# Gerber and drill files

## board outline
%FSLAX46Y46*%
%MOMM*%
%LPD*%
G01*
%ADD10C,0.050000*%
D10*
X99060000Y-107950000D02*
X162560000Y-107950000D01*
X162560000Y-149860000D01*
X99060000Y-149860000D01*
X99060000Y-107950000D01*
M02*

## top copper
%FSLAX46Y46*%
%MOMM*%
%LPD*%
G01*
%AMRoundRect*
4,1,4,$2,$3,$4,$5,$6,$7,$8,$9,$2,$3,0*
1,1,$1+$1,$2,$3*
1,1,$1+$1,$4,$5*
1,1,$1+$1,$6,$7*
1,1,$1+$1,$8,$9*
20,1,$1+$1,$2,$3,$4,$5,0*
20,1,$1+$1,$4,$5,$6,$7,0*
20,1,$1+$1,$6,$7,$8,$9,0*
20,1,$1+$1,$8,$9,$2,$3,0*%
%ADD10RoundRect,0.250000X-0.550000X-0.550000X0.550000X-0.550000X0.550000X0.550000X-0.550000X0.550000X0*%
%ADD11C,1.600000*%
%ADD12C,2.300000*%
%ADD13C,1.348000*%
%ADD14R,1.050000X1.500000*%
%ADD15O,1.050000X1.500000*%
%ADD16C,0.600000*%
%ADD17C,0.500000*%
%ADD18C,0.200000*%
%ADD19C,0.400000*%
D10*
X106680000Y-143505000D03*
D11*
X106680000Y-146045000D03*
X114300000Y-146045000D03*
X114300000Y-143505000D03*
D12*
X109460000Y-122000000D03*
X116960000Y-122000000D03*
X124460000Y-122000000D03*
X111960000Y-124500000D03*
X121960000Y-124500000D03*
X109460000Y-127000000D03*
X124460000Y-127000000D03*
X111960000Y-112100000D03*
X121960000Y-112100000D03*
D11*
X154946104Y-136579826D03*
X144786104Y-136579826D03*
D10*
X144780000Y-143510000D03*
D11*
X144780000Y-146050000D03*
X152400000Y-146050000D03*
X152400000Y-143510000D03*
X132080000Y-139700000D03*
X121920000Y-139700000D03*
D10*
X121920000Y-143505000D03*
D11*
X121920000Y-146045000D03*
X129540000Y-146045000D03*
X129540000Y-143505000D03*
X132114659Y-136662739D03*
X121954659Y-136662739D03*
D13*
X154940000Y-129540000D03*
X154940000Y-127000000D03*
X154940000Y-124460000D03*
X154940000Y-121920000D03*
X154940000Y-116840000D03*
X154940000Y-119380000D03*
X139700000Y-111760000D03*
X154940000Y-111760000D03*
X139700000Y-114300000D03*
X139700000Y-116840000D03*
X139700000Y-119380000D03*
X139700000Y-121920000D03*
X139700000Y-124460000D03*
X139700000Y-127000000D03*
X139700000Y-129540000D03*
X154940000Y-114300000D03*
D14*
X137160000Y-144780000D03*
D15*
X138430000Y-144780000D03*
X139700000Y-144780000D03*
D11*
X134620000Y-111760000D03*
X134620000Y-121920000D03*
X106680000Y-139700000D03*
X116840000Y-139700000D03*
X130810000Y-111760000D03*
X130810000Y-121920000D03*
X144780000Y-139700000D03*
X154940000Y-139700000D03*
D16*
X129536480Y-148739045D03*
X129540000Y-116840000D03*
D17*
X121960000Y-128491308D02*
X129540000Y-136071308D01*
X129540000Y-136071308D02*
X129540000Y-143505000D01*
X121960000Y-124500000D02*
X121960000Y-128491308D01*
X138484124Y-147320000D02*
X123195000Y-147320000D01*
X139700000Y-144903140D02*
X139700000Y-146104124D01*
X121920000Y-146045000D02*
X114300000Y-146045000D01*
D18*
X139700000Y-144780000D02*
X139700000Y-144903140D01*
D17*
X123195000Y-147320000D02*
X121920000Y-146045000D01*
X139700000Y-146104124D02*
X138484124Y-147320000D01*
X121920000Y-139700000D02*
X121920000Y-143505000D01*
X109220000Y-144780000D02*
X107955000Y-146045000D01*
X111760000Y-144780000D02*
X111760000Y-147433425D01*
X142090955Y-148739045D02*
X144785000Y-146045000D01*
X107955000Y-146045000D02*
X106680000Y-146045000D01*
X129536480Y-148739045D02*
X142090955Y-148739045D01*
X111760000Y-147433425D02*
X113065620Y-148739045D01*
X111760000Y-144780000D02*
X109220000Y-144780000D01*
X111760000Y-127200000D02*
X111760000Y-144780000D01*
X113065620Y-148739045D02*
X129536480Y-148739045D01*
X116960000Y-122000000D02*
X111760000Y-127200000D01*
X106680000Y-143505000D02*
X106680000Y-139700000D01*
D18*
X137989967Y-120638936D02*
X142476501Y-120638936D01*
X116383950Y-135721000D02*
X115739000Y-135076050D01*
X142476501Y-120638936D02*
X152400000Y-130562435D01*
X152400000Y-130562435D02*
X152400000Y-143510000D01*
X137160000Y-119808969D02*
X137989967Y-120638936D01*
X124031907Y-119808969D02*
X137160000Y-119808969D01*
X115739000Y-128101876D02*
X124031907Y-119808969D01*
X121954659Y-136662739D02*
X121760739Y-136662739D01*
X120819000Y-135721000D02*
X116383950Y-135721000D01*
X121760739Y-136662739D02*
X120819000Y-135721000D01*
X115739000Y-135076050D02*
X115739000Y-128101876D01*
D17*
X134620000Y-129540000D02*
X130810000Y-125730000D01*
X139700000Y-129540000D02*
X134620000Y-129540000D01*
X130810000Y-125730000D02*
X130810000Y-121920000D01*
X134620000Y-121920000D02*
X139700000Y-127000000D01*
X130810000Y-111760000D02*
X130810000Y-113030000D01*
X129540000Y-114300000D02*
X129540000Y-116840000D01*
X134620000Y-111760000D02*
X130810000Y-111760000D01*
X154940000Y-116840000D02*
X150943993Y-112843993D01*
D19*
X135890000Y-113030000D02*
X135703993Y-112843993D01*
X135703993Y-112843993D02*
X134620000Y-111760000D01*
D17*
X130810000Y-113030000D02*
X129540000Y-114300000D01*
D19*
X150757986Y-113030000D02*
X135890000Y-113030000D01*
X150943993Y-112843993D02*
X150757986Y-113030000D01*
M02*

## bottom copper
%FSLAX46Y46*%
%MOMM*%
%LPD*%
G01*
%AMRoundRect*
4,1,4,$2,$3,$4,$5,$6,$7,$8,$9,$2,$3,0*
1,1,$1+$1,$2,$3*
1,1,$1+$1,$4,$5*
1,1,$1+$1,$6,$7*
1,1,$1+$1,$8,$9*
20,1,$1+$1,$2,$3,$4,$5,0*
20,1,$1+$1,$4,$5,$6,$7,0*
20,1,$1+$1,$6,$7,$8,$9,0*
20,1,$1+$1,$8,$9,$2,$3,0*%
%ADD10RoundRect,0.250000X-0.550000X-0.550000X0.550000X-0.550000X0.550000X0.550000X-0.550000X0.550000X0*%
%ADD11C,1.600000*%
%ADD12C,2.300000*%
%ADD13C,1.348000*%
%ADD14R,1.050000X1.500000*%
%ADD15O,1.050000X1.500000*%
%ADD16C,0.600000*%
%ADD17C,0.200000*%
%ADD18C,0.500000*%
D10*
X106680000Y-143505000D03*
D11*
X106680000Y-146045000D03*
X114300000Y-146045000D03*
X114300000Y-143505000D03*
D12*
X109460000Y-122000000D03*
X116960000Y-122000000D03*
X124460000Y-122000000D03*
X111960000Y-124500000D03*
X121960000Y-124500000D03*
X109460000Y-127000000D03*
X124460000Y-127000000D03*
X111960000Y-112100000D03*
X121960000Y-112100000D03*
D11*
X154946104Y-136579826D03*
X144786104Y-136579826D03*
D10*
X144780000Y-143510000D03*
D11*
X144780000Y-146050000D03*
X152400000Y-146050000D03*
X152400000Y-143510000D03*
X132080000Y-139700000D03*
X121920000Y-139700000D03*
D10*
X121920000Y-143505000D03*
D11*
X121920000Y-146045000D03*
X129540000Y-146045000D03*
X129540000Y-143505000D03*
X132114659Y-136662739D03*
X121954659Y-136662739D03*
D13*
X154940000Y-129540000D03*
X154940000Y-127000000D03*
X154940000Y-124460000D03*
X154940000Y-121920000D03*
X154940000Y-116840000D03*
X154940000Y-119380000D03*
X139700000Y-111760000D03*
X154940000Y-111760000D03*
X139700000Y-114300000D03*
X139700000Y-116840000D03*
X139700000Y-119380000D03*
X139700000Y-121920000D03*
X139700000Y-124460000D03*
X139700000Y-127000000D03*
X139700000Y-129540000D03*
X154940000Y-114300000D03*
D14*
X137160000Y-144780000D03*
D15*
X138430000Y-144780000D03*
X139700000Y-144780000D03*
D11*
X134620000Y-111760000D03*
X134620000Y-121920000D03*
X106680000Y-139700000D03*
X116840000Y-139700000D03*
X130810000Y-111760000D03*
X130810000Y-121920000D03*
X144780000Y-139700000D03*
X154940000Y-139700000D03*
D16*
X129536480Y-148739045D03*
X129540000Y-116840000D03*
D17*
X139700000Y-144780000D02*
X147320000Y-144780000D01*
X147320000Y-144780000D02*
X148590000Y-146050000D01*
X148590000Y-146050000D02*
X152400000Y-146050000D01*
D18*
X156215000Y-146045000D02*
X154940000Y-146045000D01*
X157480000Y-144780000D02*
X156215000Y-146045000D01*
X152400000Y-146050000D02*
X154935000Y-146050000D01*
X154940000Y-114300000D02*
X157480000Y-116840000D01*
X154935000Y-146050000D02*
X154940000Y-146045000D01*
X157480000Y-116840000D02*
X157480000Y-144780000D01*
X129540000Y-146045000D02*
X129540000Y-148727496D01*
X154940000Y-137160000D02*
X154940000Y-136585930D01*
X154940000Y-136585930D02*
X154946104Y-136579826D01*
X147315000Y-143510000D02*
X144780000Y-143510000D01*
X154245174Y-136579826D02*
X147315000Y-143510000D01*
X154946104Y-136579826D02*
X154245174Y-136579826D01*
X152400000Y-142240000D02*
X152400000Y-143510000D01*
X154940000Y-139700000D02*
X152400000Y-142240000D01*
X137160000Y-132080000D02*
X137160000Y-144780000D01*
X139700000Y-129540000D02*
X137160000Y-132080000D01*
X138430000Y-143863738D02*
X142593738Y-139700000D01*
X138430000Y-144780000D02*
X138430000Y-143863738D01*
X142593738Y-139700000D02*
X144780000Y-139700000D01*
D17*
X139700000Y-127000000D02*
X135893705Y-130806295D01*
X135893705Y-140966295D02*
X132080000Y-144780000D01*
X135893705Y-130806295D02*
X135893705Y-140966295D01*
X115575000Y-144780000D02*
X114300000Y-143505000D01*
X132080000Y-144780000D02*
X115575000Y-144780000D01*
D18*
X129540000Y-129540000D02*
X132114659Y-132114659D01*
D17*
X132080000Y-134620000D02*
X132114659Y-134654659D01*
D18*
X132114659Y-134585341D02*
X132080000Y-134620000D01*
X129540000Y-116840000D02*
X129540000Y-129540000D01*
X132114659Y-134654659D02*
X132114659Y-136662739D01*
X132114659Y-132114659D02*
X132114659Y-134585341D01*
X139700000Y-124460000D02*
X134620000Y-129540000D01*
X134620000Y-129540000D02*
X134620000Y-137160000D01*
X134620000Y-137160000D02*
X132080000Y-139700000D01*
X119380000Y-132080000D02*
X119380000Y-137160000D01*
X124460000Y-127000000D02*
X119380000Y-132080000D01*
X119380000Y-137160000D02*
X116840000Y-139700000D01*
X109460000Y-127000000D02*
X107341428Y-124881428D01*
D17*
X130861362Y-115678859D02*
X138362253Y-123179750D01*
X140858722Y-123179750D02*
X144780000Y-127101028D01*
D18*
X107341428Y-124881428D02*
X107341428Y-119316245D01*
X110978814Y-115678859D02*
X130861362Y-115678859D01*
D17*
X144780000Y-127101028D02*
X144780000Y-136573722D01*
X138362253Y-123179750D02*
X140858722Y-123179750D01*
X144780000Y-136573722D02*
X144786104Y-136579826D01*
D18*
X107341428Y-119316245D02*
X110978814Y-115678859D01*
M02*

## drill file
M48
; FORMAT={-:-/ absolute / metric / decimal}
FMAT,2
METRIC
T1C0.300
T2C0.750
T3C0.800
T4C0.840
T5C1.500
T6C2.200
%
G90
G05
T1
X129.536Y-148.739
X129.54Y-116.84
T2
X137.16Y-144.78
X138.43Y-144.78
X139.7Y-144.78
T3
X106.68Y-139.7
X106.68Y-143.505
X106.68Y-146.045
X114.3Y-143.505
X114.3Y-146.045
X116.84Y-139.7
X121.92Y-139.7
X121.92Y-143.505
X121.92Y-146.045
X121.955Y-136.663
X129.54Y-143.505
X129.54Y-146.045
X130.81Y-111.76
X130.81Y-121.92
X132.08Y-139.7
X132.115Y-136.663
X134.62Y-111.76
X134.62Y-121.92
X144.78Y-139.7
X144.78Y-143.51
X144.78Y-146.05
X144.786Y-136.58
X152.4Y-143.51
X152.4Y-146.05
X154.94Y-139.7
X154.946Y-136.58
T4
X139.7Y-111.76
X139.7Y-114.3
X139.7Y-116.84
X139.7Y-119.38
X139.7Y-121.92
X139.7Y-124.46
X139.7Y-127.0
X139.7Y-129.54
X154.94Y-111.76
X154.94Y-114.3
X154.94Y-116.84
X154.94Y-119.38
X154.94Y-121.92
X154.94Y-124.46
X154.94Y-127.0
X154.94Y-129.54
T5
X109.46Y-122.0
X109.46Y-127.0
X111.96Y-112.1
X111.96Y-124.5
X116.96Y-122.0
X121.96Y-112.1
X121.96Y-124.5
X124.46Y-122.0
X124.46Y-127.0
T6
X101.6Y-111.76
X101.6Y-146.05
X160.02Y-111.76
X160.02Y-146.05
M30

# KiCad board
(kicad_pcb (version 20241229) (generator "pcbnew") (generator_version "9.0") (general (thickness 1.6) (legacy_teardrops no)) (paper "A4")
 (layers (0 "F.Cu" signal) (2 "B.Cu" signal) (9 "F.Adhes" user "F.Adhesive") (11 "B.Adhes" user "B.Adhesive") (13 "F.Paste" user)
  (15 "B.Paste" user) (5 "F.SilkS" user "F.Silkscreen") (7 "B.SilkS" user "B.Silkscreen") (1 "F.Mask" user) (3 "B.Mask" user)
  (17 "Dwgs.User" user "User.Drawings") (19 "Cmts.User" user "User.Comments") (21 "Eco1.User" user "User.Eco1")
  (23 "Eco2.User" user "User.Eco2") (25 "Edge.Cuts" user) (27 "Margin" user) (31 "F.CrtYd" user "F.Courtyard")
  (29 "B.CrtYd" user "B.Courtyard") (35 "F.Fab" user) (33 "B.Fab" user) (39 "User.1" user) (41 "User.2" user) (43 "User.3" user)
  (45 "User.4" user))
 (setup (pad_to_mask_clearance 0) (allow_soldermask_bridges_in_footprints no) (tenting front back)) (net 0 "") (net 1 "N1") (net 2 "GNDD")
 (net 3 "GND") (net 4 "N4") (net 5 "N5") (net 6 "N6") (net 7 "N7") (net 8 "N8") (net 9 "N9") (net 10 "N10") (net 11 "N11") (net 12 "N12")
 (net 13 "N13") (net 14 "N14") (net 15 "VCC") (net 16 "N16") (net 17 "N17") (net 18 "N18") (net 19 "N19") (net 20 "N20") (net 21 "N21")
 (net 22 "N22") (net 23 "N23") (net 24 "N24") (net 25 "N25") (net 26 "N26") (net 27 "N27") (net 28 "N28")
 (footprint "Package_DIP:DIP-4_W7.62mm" (layer "F.Cu") (at 106.68 143.505)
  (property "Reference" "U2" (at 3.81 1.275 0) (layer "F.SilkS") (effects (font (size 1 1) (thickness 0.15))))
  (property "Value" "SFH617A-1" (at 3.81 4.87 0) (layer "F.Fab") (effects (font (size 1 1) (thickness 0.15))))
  (pad "1" thru_hole roundrect (at 0 0) (size 1.6 1.6) (drill 0.8) (layers "*.Cu" "*.Mask") (remove_unused_layers no)
   (roundrect_rratio 0.15625) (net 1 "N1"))
  (pad "2" thru_hole circle (at 0 2.54) (size 1.6 1.6) (drill 0.8) (layers "*.Cu" "*.Mask") (remove_unused_layers no) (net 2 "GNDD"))
  (pad "3" thru_hole circle (at 7.62 2.54) (size 1.6 1.6) (drill 0.8) (layers "*.Cu" "*.Mask") (remove_unused_layers no) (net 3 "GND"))
  (pad "4" thru_hole circle (at 7.62 0) (size 1.6 1.6) (drill 0.8) (layers "*.Cu" "*.Mask") (remove_unused_layers no) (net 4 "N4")))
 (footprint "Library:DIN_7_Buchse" (layer "F.Cu") (at 116.96 124.5)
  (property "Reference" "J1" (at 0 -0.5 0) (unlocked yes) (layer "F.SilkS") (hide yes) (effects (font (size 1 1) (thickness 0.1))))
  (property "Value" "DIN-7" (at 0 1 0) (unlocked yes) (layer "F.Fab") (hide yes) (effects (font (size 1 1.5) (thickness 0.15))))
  (pad "1" thru_hole circle (at -7.5 -2.5) (size 2.3 2.3) (drill 1.5) (layers "*.Cu" "*.Mask") (remove_unused_layers no) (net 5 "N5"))
  (pad "2" thru_hole circle (at 0 -2.5) (size 2.3 2.3) (drill 1.5) (layers "*.Cu" "*.Mask") (remove_unused_layers no) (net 2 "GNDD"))
  (pad "3" thru_hole circle (at 7.5 -2.5) (size 2.3 2.3) (drill 1.5) (layers "*.Cu" "*.Mask") (remove_unused_layers no) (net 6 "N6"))
  (pad "4" thru_hole circle (at -5 0) (size 2.3 2.3) (drill 1.5) (layers "*.Cu" "*.Mask") (remove_unused_layers no) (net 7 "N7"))
  (pad "5" thru_hole circle (at 5 0) (size 2.3 2.3) (drill 1.5) (layers "*.Cu" "*.Mask") (remove_unused_layers no) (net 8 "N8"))
  (pad "6" thru_hole circle (at -7.5 2.5) (size 2.3 2.3) (drill 1.5) (layers "*.Cu" "*.Mask") (remove_unused_layers no) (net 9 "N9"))
  (pad "7" thru_hole circle (at 7.5 2.5) (size 2.3 2.3) (drill 1.5) (layers "*.Cu" "*.Mask") (remove_unused_layers no) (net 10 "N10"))
  (pad "10" thru_hole circle (at -5 -12.4) (size 2.3 2.3) (drill 1.5) (layers "*.Cu" "*.Mask") (remove_unused_layers no))
  (pad "11" thru_hole circle (at 5 -12.4) (size 2.3 2.3) (drill 1.5) (layers "*.Cu" "*.Mask") (remove_unused_layers no)))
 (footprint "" (layer "F.Cu") (at 160.02 146.05)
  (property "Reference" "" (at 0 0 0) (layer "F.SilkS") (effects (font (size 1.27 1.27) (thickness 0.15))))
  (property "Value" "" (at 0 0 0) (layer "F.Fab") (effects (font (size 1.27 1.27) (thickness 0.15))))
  (pad "" np_thru_hole circle (at 0 0) (size 2.2 2.2) (drill 2.2) (layers "*.Cu" "*.Mask")))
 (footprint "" (layer "F.Cu") (at 101.6 111.76)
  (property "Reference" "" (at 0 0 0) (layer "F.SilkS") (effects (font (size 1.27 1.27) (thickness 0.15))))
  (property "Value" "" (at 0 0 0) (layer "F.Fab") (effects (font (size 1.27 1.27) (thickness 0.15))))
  (pad "" np_thru_hole circle (at 0 0) (size 2.2 2.2) (drill 2.2) (layers "*.Cu" "*.Mask")))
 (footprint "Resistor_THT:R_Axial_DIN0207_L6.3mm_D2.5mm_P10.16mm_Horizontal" (layer "F.Cu") (at 154.946104 136.579826 180)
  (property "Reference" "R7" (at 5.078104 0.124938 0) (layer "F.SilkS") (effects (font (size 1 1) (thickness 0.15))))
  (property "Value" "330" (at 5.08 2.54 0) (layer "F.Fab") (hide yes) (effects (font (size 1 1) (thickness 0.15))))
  (pad "1" thru_hole circle (at 0 0 180) (size 1.6 1.6) (drill 0.8) (layers "*.Cu" "*.Mask") (remove_unused_layers no) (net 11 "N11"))
  (pad "2" thru_hole circle (at 10.16 0 180) (size 1.6 1.6) (drill 0.8) (layers "*.Cu" "*.Mask") (remove_unused_layers no) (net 9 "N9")))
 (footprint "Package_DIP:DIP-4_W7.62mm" (layer "F.Cu") (at 144.78 143.51)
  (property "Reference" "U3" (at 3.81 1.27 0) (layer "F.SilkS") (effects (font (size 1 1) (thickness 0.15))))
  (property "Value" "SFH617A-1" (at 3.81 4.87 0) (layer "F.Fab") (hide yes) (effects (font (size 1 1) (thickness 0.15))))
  (pad "1" thru_hole roundrect (at 0 0) (size 1.6 1.6) (drill 0.8) (layers "*.Cu" "*.Mask") (remove_unused_layers no)
   (roundrect_rratio 0.15625) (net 11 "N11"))
  (pad "2" thru_hole circle (at 0 2.54) (size 1.6 1.6) (drill 0.8) (layers "*.Cu" "*.Mask") (remove_unused_layers no) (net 2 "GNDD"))
  (pad "3" thru_hole circle (at 7.62 2.54) (size 1.6 1.6) (drill 0.8) (layers "*.Cu" "*.Mask") (remove_unused_layers no) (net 3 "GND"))
  (pad "4" thru_hole circle (at 7.62 0) (size 1.6 1.6) (drill 0.8) (layers "*.Cu" "*.Mask") (remove_unused_layers no) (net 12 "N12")))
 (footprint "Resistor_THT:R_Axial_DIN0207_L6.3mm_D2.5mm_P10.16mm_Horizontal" (layer "F.Cu") (at 132.08 139.7 180)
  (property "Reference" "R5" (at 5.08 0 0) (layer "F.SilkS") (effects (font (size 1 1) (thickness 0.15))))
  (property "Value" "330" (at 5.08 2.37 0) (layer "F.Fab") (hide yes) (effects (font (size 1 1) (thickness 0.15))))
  (pad "1" thru_hole circle (at 0 0 180) (size 1.6 1.6) (drill 0.8) (layers "*.Cu" "*.Mask") (remove_unused_layers no) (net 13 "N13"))
  (pad "2" thru_hole circle (at 10.16 0 180) (size 1.6 1.6) (drill 0.8) (layers "*.Cu" "*.Mask") (remove_unused_layers no) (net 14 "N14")))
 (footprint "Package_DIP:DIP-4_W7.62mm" (layer "F.Cu") (at 121.92 143.505)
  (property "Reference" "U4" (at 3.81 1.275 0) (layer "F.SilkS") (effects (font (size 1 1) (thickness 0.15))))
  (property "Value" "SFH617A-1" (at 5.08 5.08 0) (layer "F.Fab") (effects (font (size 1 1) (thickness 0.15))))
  (pad "1" thru_hole roundrect (at 0 0) (size 1.6 1.6) (drill 0.8) (layers "*.Cu" "*.Mask") (remove_unused_layers no)
   (roundrect_rratio 0.15625) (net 14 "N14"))
  (pad "2" thru_hole circle (at 0 2.54) (size 1.6 1.6) (drill 0.8) (layers "*.Cu" "*.Mask") (remove_unused_layers no) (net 3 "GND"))
  (pad "3" thru_hole circle (at 7.62 2.54) (size 1.6 1.6) (drill 0.8) (layers "*.Cu" "*.Mask") (remove_unused_layers no) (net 2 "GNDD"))
  (pad "4" thru_hole circle (at 7.62 0) (size 1.6 1.6) (drill 0.8) (layers "*.Cu" "*.Mask") (remove_unused_layers no) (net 8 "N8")))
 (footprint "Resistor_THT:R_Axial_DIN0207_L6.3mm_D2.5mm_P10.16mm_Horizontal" (layer "F.Cu") (at 132.114659 136.662739 180)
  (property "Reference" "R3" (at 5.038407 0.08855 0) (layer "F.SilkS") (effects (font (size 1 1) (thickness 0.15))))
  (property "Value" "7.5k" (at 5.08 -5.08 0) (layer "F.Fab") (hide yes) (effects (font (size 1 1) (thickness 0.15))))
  (pad "1" thru_hole circle (at 0 0 180) (size 1.6 1.6) (drill 0.8) (layers "*.Cu" "*.Mask") (remove_unused_layers no) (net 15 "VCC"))
  (pad "2" thru_hole circle (at 10.16 0 180) (size 1.6 1.6) (drill 0.8) (layers "*.Cu" "*.Mask") (remove_unused_layers no) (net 12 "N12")))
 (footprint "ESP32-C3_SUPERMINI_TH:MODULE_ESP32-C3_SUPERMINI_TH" (layer "F.Cu") (at 147.32 121.66)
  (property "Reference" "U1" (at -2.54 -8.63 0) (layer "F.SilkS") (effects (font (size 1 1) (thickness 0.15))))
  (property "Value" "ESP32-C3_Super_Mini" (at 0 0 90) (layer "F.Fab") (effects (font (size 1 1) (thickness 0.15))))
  (pad "0" thru_hole circle (at 7.62 7.88) (size 1.348 1.348) (drill 0.84) (layers "*.Cu" "*.Mask") (remove_unused_layers no) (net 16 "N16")
   (solder_mask_margin 0.102))
  (pad "1" thru_hole circle (at 7.62 5.34) (size 1.348 1.348) (drill 0.84) (layers "*.Cu" "*.Mask") (remove_unused_layers no) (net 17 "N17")
   (solder_mask_margin 0.102))
  (pad "2" thru_hole circle (at 7.62 2.8) (size 1.348 1.348) (drill 0.84) (layers "*.Cu" "*.Mask") (remove_unused_layers no) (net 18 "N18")
   (solder_mask_margin 0.102))
  (pad "3" thru_hole circle (at 7.62 0.26) (size 1.348 1.348) (drill 0.84) (layers "*.Cu" "*.Mask") (remove_unused_layers no) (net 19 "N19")
   (solder_mask_margin 0.102))
  (pad "3.3" thru_hole circle (at 7.62 -4.82) (size 1.348 1.348) (drill 0.84) (layers "*.Cu" "*.Mask") (remove_unused_layers no)
   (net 15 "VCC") (solder_mask_margin 0.102))
  (pad "4" thru_hole circle (at 7.62 -2.28) (size 1.348 1.348) (drill 0.84) (layers "*.Cu" "*.Mask") (remove_unused_layers no)
   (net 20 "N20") (solder_mask_margin 0.102))
  (pad "5" thru_hole circle (at -7.62 -9.9) (size 1.348 1.348) (drill 0.84) (layers "*.Cu" "*.Mask") (remove_unused_layers no)
   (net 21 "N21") (solder_mask_margin 0.102))
  (pad "5V" thru_hole circle (at 7.62 -9.9) (size 1.348 1.348) (drill 0.84) (layers "*.Cu" "*.Mask") (remove_unused_layers no)
   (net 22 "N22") (solder_mask_margin 0.102))
  (pad "6" thru_hole circle (at -7.62 -7.36) (size 1.348 1.348) (drill 0.84) (layers "*.Cu" "*.Mask") (remove_unused_layers no)
   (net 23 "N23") (solder_mask_margin 0.102))
  (pad "7" thru_hole circle (at -7.62 -4.82) (size 1.348 1.348) (drill 0.84) (layers "*.Cu" "*.Mask") (remove_unused_layers no)
   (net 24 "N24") (solder_mask_margin 0.102))
  (pad "8" thru_hole circle (at -7.62 -2.28) (size 1.348 1.348) (drill 0.84) (layers "*.Cu" "*.Mask") (remove_unused_layers no)
   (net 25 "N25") (solder_mask_margin 0.102))
  (pad "9" thru_hole circle (at -7.62 0.26) (size 1.348 1.348) (drill 0.84) (layers "*.Cu" "*.Mask") (remove_unused_layers no)
   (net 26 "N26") (solder_mask_margin 0.102))
  (pad "10" thru_hole circle (at -7.62 2.8) (size 1.348 1.348) (drill 0.84) (layers "*.Cu" "*.Mask") (remove_unused_layers no)
   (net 13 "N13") (solder_mask_margin 0.102))
  (pad "20" thru_hole circle (at -7.62 5.34) (size 1.348 1.348) (drill 0.84) (layers "*.Cu" "*.Mask") (remove_unused_layers no) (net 4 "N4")
   (solder_mask_margin 0.102))
  (pad "21" thru_hole circle (at -7.62 7.88) (size 1.348 1.348) (drill 0.84) (layers "*.Cu" "*.Mask") (remove_unused_layers no)
   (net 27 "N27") (solder_mask_margin 0.102))
  (pad "G" thru_hole circle (at 7.62 -7.36) (size 1.348 1.348) (drill 0.84) (layers "*.Cu" "*.Mask") (remove_unused_layers no) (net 3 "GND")
   (solder_mask_margin 0.102)))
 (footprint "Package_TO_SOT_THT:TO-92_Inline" (layer "F.Cu") (at 137.16 144.78)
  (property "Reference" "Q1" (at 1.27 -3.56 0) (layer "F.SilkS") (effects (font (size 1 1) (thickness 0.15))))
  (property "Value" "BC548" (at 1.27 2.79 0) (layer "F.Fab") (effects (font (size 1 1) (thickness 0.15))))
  (pad "1" thru_hole rect (at 0 0) (size 1.05 1.5) (drill 0.75) (layers "*.Cu" "*.Mask") (remove_unused_layers no) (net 27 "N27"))
  (pad "2" thru_hole oval (at 1.27 0) (size 1.05 1.5) (drill 0.75) (layers "*.Cu" "*.Mask") (remove_unused_layers no) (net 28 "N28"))
  (pad "3" thru_hole oval (at 2.54 0) (size 1.05 1.5) (drill 0.75) (layers "*.Cu" "*.Mask") (remove_unused_layers no) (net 3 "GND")))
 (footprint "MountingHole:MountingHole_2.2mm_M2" (layer "F.Cu") (at 101.6 146.05)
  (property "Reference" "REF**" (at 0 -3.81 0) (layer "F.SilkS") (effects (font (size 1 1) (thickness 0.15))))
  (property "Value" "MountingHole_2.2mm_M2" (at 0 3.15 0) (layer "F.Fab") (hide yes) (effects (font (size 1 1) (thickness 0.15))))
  (pad "" np_thru_hole circle (at 0 0) (size 2.2 2.2) (drill 2.2) (layers "*.Cu" "*.Mask")))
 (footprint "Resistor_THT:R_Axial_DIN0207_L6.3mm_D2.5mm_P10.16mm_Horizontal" (layer "F.Cu") (at 134.62 111.76 -90)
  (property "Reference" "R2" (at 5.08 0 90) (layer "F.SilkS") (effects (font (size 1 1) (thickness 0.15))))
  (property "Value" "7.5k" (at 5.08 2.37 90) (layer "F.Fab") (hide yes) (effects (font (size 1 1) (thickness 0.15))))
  (pad "1" thru_hole circle (at 0 0 270) (size 1.6 1.6) (drill 0.8) (layers "*.Cu" "*.Mask") (remove_unused_layers no) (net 15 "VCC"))
  (pad "2" thru_hole circle (at 10.16 0 270) (size 1.6 1.6) (drill 0.8) (layers "*.Cu" "*.Mask") (remove_unused_layers no) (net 4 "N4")))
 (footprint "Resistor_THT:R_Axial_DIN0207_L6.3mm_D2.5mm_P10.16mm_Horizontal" (layer "F.Cu") (at 106.68 139.7)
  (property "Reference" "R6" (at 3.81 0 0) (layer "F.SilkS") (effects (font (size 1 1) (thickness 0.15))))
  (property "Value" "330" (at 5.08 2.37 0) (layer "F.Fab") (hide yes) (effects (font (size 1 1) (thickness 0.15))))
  (pad "1" thru_hole circle (at 0 0) (size 1.6 1.6) (drill 0.8) (layers "*.Cu" "*.Mask") (remove_unused_layers no) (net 1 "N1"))
  (pad "2" thru_hole circle (at 10.16 0) (size 1.6 1.6) (drill 0.8) (layers "*.Cu" "*.Mask") (remove_unused_layers no) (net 10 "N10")))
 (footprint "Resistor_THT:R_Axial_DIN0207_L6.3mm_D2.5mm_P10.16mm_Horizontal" (layer "F.Cu") (at 130.81 111.76 -90)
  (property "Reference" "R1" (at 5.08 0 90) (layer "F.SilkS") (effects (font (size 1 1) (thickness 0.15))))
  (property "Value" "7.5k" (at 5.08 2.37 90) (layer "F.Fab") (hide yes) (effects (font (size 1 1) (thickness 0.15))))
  (pad "1" thru_hole circle (at 0 0 270) (size 1.6 1.6) (drill 0.8) (layers "*.Cu" "*.Mask") (remove_unused_layers no) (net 15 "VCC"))
  (pad "2" thru_hole circle (at 10.16 0 270) (size 1.6 1.6) (drill 0.8) (layers "*.Cu" "*.Mask") (remove_unused_layers no) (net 27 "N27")))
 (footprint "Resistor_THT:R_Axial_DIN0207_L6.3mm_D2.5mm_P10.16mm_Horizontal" (layer "F.Cu") (at 144.78 139.7)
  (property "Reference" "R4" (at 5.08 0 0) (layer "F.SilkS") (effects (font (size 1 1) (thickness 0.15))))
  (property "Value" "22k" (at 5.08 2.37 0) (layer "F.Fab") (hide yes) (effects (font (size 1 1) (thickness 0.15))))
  (pad "1" thru_hole circle (at 0 0) (size 1.6 1.6) (drill 0.8) (layers "*.Cu" "*.Mask") (remove_unused_layers no) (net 28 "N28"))
  (pad "2" thru_hole circle (at 10.16 0) (size 1.6 1.6) (drill 0.8) (layers "*.Cu" "*.Mask") (remove_unused_layers no) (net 12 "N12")))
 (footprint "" (layer "F.Cu") (at 160.02 111.76)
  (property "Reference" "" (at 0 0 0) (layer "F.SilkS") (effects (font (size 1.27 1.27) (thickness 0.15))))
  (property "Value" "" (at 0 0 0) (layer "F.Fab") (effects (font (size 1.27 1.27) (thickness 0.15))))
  (pad "" np_thru_hole circle (at 0 0) (size 2.2 2.2) (drill 2.2) (layers "*.Cu" "*.Mask")))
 (gr_rect (start 99.06 107.95) (end 162.56 149.86) (stroke (width 0.05) (type default)) (fill no) (layer "Edge.Cuts"))
 (segment (start 121.96 128.491308) (end 129.54 136.071308) (width 0.5) (layer "F.Cu") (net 8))
 (segment (start 129.54 136.071308) (end 129.54 143.505) (width 0.5) (layer "F.Cu") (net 8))
 (segment (start 121.96 124.5) (end 121.96 128.491308) (width 0.5) (layer "F.Cu") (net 8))
 (segment (start 138.484124 147.32) (end 123.195 147.32) (width 0.5) (layer "F.Cu") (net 3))
 (segment (start 139.7 144.90314) (end 139.7 146.104124) (width 0.5) (layer "F.Cu") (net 3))
 (segment (start 121.92 146.045) (end 114.3 146.045) (width 0.5) (layer "F.Cu") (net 3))
 (segment (start 139.7 144.78) (end 139.7 144.90314) (width 0.2) (layer "F.Cu") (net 3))
 (segment (start 123.195 147.32) (end 121.92 146.045) (width 0.5) (layer "F.Cu") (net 3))
 (segment (start 139.7 146.104124) (end 138.484124 147.32) (width 0.5) (layer "F.Cu") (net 3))
 (segment (start 139.7 144.78) (end 147.32 144.78) (width 0.2) (layer "B.Cu") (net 3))
 (segment (start 147.32 144.78) (end 148.59 146.05) (width 0.2) (layer "B.Cu") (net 3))
 (segment (start 148.59 146.05) (end 152.4 146.05) (width 0.2) (layer "B.Cu") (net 3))
 (segment (start 156.215 146.045) (end 154.94 146.045) (width 0.5) (layer "B.Cu") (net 3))
 (segment (start 157.48 144.78) (end 156.215 146.045) (width 0.5) (layer "B.Cu") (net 3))
 (segment (start 152.4 146.05) (end 154.935 146.05) (width 0.5) (layer "B.Cu") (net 3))
 (segment (start 154.94 114.3) (end 157.48 116.84) (width 0.5) (layer "B.Cu") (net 3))
 (segment (start 154.935 146.05) (end 154.94 146.045) (width 0.5) (layer "B.Cu") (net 3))
 (segment (start 157.48 116.84) (end 157.48 144.78) (width 0.5) (layer "B.Cu") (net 3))
 (segment (start 121.92 139.7) (end 121.92 143.505) (width 0.5) (layer "F.Cu") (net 14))
 (segment (start 109.22 144.78) (end 107.955 146.045) (width 0.5) (layer "F.Cu") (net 2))
 (segment (start 111.76 144.78) (end 111.76 147.433425) (width 0.5) (layer "F.Cu") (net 2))
 (segment (start 142.090955 148.739045) (end 144.785 146.045) (width 0.5) (layer "F.Cu") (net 2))
 (segment (start 107.955 146.045) (end 106.68 146.045) (width 0.5) (layer "F.Cu") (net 2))
 (segment (start 129.53648 148.739045) (end 142.090955 148.739045) (width 0.5) (layer "F.Cu") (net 2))
 (segment (start 111.76 147.433425) (end 113.06562 148.739045) (width 0.5) (layer "F.Cu") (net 2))
 (segment (start 111.76 144.78) (end 109.22 144.78) (width 0.5) (layer "F.Cu") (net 2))
 (segment (start 111.76 127.2) (end 111.76 144.78) (width 0.5) (layer "F.Cu") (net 2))
 (segment (start 113.06562 148.739045) (end 129.53648 148.739045) (width 0.5) (layer "F.Cu") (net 2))
 (segment (start 116.96 122) (end 111.76 127.2) (width 0.5) (layer "F.Cu") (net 2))
 (via (at 129.53648 148.739045) (size 0.6) (drill 0.3) (layers "F.Cu" "B.Cu") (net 2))
 (segment (start 129.54 146.045) (end 129.54 148.727496) (width 0.5) (layer "B.Cu") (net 2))
 (segment (start 106.68 143.505) (end 106.68 139.7) (width 0.5) (layer "F.Cu") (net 1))
 (segment (start 154.94 137.16) (end 154.94 136.58593) (width 0.5) (layer "B.Cu") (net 11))
 (segment (start 154.94 136.58593) (end 154.946104 136.579826) (width 0.5) (layer "B.Cu") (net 11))
 (segment (start 147.315 143.51) (end 144.78 143.51) (width 0.5) (layer "B.Cu") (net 11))
 (segment (start 154.245174 136.579826) (end 147.315 143.51) (width 0.5) (layer "B.Cu") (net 11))
 (segment (start 154.946104 136.579826) (end 154.245174 136.579826) (width 0.5) (layer "B.Cu") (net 11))
 (segment (start 137.989967 120.638936) (end 142.476501 120.638936) (width 0.2) (layer "F.Cu") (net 12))
 (segment (start 116.38395 135.721) (end 115.739 135.07605) (width 0.2) (layer "F.Cu") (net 12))
 (segment (start 142.476501 120.638936) (end 152.4 130.562435) (width 0.2) (layer "F.Cu") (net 12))
 (segment (start 152.4 130.562435) (end 152.4 143.51) (width 0.2) (layer "F.Cu") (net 12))
 (segment (start 137.16 119.808969) (end 137.989967 120.638936) (width 0.2) (layer "F.Cu") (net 12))
 (segment (start 124.031907 119.808969) (end 137.16 119.808969) (width 0.2) (layer "F.Cu") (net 12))
 (segment (start 115.739 128.101876) (end 124.031907 119.808969) (width 0.2) (layer "F.Cu") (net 12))
 (segment (start 121.954659 136.662739) (end 121.760739 136.662739) (width 0.2) (layer "F.Cu") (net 12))
 (segment (start 120.819 135.721) (end 116.38395 135.721) (width 0.2) (layer "F.Cu") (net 12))
 (segment (start 121.760739 136.662739) (end 120.819 135.721) (width 0.2) (layer "F.Cu") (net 12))
 (segment (start 115.739 135.07605) (end 115.739 128.101876) (width 0.2) (layer "F.Cu") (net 12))
 (segment (start 152.4 142.24) (end 152.4 143.51) (width 0.5) (layer "B.Cu") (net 12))
 (segment (start 154.94 139.7) (end 152.4 142.24) (width 0.5) (layer "B.Cu") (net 12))
 (segment (start 134.62 129.54) (end 130.81 125.73) (width 0.5) (layer "F.Cu") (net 27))
 (segment (start 139.7 129.54) (end 134.62 129.54) (width 0.5) (layer "F.Cu") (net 27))
 (segment (start 130.81 125.73) (end 130.81 121.92) (width 0.5) (layer "F.Cu") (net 27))
 (segment (start 137.16 132.08) (end 137.16 144.78) (width 0.5) (layer "B.Cu") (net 27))
 (segment (start 139.7 129.54) (end 137.16 132.08) (width 0.5) (layer "B.Cu") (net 27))
 (segment (start 138.43 143.863738) (end 142.593738 139.7) (width 0.5) (layer "B.Cu") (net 28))
 (segment (start 138.43 144.78) (end 138.43 143.863738) (width 0.5) (layer "B.Cu") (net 28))
 (segment (start 142.593738 139.7) (end 144.78 139.7) (width 0.5) (layer "B.Cu") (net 28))
 (segment (start 134.62 121.92) (end 139.7 127) (width 0.5) (layer "F.Cu") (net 4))
 (segment (start 139.7 127) (end 135.893705 130.806295) (width 0.2) (layer "B.Cu") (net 4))
 (segment (start 135.893705 140.966295) (end 132.08 144.78) (width 0.2) (layer "B.Cu") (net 4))
 (segment (start 135.893705 130.806295) (end 135.893705 140.966295) (width 0.2) (layer "B.Cu") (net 4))
 (segment (start 115.575 144.78) (end 114.3 143.505) (width 0.2) (layer "B.Cu") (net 4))
 (segment (start 132.08 144.78) (end 115.575 144.78) (width 0.2) (layer "B.Cu") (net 4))
 (segment (start 130.81 111.76) (end 130.81 113.03) (width 0.5) (layer "F.Cu") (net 15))
 (segment (start 129.54 114.3) (end 129.54 116.84) (width 0.5) (layer "F.Cu") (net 15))
 (segment (start 134.62 111.76) (end 130.81 111.76) (width 0.5) (layer "F.Cu") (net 15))
 (segment (start 154.94 116.84) (end 150.943993 112.843993) (width 0.5) (layer "F.Cu") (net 15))
 (segment (start 135.89 113.03) (end 135.703993 112.843993) (width 0.4) (layer "F.Cu") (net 15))
 (segment (start 135.703993 112.843993) (end 134.62 111.76) (width 0.4) (layer "F.Cu") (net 15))
 (segment (start 130.81 113.03) (end 129.54 114.3) (width 0.5) (layer "F.Cu") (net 15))
 (segment (start 150.757986 113.03) (end 135.89 113.03) (width 0.4) (layer "F.Cu") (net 15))
 (segment (start 150.943993 112.843993) (end 150.757986 113.03) (width 0.4) (layer "F.Cu") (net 15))
 (via (at 129.54 116.84) (size 0.6) (drill 0.3) (layers "F.Cu" "B.Cu") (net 15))
 (segment (start 129.54 129.54) (end 132.114659 132.114659) (width 0.5) (layer "B.Cu") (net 15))
 (segment (start 132.08 134.62) (end 132.114659 134.654659) (width 0.2) (layer "B.Cu") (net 15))
 (segment (start 132.114659 134.585341) (end 132.08 134.62) (width 0.5) (layer "B.Cu") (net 15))
 (segment (start 129.54 116.84) (end 129.54 129.54) (width 0.5) (layer "B.Cu") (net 15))
 (segment (start 132.114659 134.654659) (end 132.114659 136.662739) (width 0.5) (layer "B.Cu") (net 15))
 (segment (start 132.114659 132.114659) (end 132.114659 134.585341) (width 0.5) (layer "B.Cu") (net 15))
 (segment (start 139.7 124.46) (end 134.62 129.54) (width 0.5) (layer "B.Cu") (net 13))
 (segment (start 134.62 129.54) (end 134.62 137.16) (width 0.5) (layer "B.Cu") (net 13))
 (segment (start 134.62 137.16) (end 132.08 139.7) (width 0.5) (layer "B.Cu") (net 13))
 (segment (start 119.38 132.08) (end 119.38 137.16) (width 0.5) (layer "B.Cu") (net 10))
 (segment (start 124.46 127) (end 119.38 132.08) (width 0.5) (layer "B.Cu") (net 10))
 (segment (start 119.38 137.16) (end 116.84 139.7) (width 0.5) (layer "B.Cu") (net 10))
 (segment (start 109.46 127) (end 107.341428 124.881428) (width 0.5) (layer "B.Cu") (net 9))
 (segment (start 130.861362 115.678859) (end 138.362253 123.17975) (width 0.2) (layer "B.Cu") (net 9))
 (segment (start 140.858722 123.17975) (end 144.78 127.101028) (width 0.2) (layer "B.Cu") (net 9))
 (segment (start 107.341428 124.881428) (end 107.341428 119.316245) (width 0.5) (layer "B.Cu") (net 9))
 (segment (start 110.978814 115.678859) (end 130.861362 115.678859) (width 0.5) (layer "B.Cu") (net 9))
 (segment (start 144.78 127.101028) (end 144.78 136.573722) (width 0.2) (layer "B.Cu") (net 9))
 (segment (start 138.362253 123.17975) (end 140.858722 123.17975) (width 0.2) (layer "B.Cu") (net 9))
 (segment (start 144.78 136.573722) (end 144.786104 136.579826) (width 0.2) (layer "B.Cu") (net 9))
 (segment (start 107.341428 119.316245) (end 110.978814 115.678859) (width 0.5) (layer "B.Cu") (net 9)))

